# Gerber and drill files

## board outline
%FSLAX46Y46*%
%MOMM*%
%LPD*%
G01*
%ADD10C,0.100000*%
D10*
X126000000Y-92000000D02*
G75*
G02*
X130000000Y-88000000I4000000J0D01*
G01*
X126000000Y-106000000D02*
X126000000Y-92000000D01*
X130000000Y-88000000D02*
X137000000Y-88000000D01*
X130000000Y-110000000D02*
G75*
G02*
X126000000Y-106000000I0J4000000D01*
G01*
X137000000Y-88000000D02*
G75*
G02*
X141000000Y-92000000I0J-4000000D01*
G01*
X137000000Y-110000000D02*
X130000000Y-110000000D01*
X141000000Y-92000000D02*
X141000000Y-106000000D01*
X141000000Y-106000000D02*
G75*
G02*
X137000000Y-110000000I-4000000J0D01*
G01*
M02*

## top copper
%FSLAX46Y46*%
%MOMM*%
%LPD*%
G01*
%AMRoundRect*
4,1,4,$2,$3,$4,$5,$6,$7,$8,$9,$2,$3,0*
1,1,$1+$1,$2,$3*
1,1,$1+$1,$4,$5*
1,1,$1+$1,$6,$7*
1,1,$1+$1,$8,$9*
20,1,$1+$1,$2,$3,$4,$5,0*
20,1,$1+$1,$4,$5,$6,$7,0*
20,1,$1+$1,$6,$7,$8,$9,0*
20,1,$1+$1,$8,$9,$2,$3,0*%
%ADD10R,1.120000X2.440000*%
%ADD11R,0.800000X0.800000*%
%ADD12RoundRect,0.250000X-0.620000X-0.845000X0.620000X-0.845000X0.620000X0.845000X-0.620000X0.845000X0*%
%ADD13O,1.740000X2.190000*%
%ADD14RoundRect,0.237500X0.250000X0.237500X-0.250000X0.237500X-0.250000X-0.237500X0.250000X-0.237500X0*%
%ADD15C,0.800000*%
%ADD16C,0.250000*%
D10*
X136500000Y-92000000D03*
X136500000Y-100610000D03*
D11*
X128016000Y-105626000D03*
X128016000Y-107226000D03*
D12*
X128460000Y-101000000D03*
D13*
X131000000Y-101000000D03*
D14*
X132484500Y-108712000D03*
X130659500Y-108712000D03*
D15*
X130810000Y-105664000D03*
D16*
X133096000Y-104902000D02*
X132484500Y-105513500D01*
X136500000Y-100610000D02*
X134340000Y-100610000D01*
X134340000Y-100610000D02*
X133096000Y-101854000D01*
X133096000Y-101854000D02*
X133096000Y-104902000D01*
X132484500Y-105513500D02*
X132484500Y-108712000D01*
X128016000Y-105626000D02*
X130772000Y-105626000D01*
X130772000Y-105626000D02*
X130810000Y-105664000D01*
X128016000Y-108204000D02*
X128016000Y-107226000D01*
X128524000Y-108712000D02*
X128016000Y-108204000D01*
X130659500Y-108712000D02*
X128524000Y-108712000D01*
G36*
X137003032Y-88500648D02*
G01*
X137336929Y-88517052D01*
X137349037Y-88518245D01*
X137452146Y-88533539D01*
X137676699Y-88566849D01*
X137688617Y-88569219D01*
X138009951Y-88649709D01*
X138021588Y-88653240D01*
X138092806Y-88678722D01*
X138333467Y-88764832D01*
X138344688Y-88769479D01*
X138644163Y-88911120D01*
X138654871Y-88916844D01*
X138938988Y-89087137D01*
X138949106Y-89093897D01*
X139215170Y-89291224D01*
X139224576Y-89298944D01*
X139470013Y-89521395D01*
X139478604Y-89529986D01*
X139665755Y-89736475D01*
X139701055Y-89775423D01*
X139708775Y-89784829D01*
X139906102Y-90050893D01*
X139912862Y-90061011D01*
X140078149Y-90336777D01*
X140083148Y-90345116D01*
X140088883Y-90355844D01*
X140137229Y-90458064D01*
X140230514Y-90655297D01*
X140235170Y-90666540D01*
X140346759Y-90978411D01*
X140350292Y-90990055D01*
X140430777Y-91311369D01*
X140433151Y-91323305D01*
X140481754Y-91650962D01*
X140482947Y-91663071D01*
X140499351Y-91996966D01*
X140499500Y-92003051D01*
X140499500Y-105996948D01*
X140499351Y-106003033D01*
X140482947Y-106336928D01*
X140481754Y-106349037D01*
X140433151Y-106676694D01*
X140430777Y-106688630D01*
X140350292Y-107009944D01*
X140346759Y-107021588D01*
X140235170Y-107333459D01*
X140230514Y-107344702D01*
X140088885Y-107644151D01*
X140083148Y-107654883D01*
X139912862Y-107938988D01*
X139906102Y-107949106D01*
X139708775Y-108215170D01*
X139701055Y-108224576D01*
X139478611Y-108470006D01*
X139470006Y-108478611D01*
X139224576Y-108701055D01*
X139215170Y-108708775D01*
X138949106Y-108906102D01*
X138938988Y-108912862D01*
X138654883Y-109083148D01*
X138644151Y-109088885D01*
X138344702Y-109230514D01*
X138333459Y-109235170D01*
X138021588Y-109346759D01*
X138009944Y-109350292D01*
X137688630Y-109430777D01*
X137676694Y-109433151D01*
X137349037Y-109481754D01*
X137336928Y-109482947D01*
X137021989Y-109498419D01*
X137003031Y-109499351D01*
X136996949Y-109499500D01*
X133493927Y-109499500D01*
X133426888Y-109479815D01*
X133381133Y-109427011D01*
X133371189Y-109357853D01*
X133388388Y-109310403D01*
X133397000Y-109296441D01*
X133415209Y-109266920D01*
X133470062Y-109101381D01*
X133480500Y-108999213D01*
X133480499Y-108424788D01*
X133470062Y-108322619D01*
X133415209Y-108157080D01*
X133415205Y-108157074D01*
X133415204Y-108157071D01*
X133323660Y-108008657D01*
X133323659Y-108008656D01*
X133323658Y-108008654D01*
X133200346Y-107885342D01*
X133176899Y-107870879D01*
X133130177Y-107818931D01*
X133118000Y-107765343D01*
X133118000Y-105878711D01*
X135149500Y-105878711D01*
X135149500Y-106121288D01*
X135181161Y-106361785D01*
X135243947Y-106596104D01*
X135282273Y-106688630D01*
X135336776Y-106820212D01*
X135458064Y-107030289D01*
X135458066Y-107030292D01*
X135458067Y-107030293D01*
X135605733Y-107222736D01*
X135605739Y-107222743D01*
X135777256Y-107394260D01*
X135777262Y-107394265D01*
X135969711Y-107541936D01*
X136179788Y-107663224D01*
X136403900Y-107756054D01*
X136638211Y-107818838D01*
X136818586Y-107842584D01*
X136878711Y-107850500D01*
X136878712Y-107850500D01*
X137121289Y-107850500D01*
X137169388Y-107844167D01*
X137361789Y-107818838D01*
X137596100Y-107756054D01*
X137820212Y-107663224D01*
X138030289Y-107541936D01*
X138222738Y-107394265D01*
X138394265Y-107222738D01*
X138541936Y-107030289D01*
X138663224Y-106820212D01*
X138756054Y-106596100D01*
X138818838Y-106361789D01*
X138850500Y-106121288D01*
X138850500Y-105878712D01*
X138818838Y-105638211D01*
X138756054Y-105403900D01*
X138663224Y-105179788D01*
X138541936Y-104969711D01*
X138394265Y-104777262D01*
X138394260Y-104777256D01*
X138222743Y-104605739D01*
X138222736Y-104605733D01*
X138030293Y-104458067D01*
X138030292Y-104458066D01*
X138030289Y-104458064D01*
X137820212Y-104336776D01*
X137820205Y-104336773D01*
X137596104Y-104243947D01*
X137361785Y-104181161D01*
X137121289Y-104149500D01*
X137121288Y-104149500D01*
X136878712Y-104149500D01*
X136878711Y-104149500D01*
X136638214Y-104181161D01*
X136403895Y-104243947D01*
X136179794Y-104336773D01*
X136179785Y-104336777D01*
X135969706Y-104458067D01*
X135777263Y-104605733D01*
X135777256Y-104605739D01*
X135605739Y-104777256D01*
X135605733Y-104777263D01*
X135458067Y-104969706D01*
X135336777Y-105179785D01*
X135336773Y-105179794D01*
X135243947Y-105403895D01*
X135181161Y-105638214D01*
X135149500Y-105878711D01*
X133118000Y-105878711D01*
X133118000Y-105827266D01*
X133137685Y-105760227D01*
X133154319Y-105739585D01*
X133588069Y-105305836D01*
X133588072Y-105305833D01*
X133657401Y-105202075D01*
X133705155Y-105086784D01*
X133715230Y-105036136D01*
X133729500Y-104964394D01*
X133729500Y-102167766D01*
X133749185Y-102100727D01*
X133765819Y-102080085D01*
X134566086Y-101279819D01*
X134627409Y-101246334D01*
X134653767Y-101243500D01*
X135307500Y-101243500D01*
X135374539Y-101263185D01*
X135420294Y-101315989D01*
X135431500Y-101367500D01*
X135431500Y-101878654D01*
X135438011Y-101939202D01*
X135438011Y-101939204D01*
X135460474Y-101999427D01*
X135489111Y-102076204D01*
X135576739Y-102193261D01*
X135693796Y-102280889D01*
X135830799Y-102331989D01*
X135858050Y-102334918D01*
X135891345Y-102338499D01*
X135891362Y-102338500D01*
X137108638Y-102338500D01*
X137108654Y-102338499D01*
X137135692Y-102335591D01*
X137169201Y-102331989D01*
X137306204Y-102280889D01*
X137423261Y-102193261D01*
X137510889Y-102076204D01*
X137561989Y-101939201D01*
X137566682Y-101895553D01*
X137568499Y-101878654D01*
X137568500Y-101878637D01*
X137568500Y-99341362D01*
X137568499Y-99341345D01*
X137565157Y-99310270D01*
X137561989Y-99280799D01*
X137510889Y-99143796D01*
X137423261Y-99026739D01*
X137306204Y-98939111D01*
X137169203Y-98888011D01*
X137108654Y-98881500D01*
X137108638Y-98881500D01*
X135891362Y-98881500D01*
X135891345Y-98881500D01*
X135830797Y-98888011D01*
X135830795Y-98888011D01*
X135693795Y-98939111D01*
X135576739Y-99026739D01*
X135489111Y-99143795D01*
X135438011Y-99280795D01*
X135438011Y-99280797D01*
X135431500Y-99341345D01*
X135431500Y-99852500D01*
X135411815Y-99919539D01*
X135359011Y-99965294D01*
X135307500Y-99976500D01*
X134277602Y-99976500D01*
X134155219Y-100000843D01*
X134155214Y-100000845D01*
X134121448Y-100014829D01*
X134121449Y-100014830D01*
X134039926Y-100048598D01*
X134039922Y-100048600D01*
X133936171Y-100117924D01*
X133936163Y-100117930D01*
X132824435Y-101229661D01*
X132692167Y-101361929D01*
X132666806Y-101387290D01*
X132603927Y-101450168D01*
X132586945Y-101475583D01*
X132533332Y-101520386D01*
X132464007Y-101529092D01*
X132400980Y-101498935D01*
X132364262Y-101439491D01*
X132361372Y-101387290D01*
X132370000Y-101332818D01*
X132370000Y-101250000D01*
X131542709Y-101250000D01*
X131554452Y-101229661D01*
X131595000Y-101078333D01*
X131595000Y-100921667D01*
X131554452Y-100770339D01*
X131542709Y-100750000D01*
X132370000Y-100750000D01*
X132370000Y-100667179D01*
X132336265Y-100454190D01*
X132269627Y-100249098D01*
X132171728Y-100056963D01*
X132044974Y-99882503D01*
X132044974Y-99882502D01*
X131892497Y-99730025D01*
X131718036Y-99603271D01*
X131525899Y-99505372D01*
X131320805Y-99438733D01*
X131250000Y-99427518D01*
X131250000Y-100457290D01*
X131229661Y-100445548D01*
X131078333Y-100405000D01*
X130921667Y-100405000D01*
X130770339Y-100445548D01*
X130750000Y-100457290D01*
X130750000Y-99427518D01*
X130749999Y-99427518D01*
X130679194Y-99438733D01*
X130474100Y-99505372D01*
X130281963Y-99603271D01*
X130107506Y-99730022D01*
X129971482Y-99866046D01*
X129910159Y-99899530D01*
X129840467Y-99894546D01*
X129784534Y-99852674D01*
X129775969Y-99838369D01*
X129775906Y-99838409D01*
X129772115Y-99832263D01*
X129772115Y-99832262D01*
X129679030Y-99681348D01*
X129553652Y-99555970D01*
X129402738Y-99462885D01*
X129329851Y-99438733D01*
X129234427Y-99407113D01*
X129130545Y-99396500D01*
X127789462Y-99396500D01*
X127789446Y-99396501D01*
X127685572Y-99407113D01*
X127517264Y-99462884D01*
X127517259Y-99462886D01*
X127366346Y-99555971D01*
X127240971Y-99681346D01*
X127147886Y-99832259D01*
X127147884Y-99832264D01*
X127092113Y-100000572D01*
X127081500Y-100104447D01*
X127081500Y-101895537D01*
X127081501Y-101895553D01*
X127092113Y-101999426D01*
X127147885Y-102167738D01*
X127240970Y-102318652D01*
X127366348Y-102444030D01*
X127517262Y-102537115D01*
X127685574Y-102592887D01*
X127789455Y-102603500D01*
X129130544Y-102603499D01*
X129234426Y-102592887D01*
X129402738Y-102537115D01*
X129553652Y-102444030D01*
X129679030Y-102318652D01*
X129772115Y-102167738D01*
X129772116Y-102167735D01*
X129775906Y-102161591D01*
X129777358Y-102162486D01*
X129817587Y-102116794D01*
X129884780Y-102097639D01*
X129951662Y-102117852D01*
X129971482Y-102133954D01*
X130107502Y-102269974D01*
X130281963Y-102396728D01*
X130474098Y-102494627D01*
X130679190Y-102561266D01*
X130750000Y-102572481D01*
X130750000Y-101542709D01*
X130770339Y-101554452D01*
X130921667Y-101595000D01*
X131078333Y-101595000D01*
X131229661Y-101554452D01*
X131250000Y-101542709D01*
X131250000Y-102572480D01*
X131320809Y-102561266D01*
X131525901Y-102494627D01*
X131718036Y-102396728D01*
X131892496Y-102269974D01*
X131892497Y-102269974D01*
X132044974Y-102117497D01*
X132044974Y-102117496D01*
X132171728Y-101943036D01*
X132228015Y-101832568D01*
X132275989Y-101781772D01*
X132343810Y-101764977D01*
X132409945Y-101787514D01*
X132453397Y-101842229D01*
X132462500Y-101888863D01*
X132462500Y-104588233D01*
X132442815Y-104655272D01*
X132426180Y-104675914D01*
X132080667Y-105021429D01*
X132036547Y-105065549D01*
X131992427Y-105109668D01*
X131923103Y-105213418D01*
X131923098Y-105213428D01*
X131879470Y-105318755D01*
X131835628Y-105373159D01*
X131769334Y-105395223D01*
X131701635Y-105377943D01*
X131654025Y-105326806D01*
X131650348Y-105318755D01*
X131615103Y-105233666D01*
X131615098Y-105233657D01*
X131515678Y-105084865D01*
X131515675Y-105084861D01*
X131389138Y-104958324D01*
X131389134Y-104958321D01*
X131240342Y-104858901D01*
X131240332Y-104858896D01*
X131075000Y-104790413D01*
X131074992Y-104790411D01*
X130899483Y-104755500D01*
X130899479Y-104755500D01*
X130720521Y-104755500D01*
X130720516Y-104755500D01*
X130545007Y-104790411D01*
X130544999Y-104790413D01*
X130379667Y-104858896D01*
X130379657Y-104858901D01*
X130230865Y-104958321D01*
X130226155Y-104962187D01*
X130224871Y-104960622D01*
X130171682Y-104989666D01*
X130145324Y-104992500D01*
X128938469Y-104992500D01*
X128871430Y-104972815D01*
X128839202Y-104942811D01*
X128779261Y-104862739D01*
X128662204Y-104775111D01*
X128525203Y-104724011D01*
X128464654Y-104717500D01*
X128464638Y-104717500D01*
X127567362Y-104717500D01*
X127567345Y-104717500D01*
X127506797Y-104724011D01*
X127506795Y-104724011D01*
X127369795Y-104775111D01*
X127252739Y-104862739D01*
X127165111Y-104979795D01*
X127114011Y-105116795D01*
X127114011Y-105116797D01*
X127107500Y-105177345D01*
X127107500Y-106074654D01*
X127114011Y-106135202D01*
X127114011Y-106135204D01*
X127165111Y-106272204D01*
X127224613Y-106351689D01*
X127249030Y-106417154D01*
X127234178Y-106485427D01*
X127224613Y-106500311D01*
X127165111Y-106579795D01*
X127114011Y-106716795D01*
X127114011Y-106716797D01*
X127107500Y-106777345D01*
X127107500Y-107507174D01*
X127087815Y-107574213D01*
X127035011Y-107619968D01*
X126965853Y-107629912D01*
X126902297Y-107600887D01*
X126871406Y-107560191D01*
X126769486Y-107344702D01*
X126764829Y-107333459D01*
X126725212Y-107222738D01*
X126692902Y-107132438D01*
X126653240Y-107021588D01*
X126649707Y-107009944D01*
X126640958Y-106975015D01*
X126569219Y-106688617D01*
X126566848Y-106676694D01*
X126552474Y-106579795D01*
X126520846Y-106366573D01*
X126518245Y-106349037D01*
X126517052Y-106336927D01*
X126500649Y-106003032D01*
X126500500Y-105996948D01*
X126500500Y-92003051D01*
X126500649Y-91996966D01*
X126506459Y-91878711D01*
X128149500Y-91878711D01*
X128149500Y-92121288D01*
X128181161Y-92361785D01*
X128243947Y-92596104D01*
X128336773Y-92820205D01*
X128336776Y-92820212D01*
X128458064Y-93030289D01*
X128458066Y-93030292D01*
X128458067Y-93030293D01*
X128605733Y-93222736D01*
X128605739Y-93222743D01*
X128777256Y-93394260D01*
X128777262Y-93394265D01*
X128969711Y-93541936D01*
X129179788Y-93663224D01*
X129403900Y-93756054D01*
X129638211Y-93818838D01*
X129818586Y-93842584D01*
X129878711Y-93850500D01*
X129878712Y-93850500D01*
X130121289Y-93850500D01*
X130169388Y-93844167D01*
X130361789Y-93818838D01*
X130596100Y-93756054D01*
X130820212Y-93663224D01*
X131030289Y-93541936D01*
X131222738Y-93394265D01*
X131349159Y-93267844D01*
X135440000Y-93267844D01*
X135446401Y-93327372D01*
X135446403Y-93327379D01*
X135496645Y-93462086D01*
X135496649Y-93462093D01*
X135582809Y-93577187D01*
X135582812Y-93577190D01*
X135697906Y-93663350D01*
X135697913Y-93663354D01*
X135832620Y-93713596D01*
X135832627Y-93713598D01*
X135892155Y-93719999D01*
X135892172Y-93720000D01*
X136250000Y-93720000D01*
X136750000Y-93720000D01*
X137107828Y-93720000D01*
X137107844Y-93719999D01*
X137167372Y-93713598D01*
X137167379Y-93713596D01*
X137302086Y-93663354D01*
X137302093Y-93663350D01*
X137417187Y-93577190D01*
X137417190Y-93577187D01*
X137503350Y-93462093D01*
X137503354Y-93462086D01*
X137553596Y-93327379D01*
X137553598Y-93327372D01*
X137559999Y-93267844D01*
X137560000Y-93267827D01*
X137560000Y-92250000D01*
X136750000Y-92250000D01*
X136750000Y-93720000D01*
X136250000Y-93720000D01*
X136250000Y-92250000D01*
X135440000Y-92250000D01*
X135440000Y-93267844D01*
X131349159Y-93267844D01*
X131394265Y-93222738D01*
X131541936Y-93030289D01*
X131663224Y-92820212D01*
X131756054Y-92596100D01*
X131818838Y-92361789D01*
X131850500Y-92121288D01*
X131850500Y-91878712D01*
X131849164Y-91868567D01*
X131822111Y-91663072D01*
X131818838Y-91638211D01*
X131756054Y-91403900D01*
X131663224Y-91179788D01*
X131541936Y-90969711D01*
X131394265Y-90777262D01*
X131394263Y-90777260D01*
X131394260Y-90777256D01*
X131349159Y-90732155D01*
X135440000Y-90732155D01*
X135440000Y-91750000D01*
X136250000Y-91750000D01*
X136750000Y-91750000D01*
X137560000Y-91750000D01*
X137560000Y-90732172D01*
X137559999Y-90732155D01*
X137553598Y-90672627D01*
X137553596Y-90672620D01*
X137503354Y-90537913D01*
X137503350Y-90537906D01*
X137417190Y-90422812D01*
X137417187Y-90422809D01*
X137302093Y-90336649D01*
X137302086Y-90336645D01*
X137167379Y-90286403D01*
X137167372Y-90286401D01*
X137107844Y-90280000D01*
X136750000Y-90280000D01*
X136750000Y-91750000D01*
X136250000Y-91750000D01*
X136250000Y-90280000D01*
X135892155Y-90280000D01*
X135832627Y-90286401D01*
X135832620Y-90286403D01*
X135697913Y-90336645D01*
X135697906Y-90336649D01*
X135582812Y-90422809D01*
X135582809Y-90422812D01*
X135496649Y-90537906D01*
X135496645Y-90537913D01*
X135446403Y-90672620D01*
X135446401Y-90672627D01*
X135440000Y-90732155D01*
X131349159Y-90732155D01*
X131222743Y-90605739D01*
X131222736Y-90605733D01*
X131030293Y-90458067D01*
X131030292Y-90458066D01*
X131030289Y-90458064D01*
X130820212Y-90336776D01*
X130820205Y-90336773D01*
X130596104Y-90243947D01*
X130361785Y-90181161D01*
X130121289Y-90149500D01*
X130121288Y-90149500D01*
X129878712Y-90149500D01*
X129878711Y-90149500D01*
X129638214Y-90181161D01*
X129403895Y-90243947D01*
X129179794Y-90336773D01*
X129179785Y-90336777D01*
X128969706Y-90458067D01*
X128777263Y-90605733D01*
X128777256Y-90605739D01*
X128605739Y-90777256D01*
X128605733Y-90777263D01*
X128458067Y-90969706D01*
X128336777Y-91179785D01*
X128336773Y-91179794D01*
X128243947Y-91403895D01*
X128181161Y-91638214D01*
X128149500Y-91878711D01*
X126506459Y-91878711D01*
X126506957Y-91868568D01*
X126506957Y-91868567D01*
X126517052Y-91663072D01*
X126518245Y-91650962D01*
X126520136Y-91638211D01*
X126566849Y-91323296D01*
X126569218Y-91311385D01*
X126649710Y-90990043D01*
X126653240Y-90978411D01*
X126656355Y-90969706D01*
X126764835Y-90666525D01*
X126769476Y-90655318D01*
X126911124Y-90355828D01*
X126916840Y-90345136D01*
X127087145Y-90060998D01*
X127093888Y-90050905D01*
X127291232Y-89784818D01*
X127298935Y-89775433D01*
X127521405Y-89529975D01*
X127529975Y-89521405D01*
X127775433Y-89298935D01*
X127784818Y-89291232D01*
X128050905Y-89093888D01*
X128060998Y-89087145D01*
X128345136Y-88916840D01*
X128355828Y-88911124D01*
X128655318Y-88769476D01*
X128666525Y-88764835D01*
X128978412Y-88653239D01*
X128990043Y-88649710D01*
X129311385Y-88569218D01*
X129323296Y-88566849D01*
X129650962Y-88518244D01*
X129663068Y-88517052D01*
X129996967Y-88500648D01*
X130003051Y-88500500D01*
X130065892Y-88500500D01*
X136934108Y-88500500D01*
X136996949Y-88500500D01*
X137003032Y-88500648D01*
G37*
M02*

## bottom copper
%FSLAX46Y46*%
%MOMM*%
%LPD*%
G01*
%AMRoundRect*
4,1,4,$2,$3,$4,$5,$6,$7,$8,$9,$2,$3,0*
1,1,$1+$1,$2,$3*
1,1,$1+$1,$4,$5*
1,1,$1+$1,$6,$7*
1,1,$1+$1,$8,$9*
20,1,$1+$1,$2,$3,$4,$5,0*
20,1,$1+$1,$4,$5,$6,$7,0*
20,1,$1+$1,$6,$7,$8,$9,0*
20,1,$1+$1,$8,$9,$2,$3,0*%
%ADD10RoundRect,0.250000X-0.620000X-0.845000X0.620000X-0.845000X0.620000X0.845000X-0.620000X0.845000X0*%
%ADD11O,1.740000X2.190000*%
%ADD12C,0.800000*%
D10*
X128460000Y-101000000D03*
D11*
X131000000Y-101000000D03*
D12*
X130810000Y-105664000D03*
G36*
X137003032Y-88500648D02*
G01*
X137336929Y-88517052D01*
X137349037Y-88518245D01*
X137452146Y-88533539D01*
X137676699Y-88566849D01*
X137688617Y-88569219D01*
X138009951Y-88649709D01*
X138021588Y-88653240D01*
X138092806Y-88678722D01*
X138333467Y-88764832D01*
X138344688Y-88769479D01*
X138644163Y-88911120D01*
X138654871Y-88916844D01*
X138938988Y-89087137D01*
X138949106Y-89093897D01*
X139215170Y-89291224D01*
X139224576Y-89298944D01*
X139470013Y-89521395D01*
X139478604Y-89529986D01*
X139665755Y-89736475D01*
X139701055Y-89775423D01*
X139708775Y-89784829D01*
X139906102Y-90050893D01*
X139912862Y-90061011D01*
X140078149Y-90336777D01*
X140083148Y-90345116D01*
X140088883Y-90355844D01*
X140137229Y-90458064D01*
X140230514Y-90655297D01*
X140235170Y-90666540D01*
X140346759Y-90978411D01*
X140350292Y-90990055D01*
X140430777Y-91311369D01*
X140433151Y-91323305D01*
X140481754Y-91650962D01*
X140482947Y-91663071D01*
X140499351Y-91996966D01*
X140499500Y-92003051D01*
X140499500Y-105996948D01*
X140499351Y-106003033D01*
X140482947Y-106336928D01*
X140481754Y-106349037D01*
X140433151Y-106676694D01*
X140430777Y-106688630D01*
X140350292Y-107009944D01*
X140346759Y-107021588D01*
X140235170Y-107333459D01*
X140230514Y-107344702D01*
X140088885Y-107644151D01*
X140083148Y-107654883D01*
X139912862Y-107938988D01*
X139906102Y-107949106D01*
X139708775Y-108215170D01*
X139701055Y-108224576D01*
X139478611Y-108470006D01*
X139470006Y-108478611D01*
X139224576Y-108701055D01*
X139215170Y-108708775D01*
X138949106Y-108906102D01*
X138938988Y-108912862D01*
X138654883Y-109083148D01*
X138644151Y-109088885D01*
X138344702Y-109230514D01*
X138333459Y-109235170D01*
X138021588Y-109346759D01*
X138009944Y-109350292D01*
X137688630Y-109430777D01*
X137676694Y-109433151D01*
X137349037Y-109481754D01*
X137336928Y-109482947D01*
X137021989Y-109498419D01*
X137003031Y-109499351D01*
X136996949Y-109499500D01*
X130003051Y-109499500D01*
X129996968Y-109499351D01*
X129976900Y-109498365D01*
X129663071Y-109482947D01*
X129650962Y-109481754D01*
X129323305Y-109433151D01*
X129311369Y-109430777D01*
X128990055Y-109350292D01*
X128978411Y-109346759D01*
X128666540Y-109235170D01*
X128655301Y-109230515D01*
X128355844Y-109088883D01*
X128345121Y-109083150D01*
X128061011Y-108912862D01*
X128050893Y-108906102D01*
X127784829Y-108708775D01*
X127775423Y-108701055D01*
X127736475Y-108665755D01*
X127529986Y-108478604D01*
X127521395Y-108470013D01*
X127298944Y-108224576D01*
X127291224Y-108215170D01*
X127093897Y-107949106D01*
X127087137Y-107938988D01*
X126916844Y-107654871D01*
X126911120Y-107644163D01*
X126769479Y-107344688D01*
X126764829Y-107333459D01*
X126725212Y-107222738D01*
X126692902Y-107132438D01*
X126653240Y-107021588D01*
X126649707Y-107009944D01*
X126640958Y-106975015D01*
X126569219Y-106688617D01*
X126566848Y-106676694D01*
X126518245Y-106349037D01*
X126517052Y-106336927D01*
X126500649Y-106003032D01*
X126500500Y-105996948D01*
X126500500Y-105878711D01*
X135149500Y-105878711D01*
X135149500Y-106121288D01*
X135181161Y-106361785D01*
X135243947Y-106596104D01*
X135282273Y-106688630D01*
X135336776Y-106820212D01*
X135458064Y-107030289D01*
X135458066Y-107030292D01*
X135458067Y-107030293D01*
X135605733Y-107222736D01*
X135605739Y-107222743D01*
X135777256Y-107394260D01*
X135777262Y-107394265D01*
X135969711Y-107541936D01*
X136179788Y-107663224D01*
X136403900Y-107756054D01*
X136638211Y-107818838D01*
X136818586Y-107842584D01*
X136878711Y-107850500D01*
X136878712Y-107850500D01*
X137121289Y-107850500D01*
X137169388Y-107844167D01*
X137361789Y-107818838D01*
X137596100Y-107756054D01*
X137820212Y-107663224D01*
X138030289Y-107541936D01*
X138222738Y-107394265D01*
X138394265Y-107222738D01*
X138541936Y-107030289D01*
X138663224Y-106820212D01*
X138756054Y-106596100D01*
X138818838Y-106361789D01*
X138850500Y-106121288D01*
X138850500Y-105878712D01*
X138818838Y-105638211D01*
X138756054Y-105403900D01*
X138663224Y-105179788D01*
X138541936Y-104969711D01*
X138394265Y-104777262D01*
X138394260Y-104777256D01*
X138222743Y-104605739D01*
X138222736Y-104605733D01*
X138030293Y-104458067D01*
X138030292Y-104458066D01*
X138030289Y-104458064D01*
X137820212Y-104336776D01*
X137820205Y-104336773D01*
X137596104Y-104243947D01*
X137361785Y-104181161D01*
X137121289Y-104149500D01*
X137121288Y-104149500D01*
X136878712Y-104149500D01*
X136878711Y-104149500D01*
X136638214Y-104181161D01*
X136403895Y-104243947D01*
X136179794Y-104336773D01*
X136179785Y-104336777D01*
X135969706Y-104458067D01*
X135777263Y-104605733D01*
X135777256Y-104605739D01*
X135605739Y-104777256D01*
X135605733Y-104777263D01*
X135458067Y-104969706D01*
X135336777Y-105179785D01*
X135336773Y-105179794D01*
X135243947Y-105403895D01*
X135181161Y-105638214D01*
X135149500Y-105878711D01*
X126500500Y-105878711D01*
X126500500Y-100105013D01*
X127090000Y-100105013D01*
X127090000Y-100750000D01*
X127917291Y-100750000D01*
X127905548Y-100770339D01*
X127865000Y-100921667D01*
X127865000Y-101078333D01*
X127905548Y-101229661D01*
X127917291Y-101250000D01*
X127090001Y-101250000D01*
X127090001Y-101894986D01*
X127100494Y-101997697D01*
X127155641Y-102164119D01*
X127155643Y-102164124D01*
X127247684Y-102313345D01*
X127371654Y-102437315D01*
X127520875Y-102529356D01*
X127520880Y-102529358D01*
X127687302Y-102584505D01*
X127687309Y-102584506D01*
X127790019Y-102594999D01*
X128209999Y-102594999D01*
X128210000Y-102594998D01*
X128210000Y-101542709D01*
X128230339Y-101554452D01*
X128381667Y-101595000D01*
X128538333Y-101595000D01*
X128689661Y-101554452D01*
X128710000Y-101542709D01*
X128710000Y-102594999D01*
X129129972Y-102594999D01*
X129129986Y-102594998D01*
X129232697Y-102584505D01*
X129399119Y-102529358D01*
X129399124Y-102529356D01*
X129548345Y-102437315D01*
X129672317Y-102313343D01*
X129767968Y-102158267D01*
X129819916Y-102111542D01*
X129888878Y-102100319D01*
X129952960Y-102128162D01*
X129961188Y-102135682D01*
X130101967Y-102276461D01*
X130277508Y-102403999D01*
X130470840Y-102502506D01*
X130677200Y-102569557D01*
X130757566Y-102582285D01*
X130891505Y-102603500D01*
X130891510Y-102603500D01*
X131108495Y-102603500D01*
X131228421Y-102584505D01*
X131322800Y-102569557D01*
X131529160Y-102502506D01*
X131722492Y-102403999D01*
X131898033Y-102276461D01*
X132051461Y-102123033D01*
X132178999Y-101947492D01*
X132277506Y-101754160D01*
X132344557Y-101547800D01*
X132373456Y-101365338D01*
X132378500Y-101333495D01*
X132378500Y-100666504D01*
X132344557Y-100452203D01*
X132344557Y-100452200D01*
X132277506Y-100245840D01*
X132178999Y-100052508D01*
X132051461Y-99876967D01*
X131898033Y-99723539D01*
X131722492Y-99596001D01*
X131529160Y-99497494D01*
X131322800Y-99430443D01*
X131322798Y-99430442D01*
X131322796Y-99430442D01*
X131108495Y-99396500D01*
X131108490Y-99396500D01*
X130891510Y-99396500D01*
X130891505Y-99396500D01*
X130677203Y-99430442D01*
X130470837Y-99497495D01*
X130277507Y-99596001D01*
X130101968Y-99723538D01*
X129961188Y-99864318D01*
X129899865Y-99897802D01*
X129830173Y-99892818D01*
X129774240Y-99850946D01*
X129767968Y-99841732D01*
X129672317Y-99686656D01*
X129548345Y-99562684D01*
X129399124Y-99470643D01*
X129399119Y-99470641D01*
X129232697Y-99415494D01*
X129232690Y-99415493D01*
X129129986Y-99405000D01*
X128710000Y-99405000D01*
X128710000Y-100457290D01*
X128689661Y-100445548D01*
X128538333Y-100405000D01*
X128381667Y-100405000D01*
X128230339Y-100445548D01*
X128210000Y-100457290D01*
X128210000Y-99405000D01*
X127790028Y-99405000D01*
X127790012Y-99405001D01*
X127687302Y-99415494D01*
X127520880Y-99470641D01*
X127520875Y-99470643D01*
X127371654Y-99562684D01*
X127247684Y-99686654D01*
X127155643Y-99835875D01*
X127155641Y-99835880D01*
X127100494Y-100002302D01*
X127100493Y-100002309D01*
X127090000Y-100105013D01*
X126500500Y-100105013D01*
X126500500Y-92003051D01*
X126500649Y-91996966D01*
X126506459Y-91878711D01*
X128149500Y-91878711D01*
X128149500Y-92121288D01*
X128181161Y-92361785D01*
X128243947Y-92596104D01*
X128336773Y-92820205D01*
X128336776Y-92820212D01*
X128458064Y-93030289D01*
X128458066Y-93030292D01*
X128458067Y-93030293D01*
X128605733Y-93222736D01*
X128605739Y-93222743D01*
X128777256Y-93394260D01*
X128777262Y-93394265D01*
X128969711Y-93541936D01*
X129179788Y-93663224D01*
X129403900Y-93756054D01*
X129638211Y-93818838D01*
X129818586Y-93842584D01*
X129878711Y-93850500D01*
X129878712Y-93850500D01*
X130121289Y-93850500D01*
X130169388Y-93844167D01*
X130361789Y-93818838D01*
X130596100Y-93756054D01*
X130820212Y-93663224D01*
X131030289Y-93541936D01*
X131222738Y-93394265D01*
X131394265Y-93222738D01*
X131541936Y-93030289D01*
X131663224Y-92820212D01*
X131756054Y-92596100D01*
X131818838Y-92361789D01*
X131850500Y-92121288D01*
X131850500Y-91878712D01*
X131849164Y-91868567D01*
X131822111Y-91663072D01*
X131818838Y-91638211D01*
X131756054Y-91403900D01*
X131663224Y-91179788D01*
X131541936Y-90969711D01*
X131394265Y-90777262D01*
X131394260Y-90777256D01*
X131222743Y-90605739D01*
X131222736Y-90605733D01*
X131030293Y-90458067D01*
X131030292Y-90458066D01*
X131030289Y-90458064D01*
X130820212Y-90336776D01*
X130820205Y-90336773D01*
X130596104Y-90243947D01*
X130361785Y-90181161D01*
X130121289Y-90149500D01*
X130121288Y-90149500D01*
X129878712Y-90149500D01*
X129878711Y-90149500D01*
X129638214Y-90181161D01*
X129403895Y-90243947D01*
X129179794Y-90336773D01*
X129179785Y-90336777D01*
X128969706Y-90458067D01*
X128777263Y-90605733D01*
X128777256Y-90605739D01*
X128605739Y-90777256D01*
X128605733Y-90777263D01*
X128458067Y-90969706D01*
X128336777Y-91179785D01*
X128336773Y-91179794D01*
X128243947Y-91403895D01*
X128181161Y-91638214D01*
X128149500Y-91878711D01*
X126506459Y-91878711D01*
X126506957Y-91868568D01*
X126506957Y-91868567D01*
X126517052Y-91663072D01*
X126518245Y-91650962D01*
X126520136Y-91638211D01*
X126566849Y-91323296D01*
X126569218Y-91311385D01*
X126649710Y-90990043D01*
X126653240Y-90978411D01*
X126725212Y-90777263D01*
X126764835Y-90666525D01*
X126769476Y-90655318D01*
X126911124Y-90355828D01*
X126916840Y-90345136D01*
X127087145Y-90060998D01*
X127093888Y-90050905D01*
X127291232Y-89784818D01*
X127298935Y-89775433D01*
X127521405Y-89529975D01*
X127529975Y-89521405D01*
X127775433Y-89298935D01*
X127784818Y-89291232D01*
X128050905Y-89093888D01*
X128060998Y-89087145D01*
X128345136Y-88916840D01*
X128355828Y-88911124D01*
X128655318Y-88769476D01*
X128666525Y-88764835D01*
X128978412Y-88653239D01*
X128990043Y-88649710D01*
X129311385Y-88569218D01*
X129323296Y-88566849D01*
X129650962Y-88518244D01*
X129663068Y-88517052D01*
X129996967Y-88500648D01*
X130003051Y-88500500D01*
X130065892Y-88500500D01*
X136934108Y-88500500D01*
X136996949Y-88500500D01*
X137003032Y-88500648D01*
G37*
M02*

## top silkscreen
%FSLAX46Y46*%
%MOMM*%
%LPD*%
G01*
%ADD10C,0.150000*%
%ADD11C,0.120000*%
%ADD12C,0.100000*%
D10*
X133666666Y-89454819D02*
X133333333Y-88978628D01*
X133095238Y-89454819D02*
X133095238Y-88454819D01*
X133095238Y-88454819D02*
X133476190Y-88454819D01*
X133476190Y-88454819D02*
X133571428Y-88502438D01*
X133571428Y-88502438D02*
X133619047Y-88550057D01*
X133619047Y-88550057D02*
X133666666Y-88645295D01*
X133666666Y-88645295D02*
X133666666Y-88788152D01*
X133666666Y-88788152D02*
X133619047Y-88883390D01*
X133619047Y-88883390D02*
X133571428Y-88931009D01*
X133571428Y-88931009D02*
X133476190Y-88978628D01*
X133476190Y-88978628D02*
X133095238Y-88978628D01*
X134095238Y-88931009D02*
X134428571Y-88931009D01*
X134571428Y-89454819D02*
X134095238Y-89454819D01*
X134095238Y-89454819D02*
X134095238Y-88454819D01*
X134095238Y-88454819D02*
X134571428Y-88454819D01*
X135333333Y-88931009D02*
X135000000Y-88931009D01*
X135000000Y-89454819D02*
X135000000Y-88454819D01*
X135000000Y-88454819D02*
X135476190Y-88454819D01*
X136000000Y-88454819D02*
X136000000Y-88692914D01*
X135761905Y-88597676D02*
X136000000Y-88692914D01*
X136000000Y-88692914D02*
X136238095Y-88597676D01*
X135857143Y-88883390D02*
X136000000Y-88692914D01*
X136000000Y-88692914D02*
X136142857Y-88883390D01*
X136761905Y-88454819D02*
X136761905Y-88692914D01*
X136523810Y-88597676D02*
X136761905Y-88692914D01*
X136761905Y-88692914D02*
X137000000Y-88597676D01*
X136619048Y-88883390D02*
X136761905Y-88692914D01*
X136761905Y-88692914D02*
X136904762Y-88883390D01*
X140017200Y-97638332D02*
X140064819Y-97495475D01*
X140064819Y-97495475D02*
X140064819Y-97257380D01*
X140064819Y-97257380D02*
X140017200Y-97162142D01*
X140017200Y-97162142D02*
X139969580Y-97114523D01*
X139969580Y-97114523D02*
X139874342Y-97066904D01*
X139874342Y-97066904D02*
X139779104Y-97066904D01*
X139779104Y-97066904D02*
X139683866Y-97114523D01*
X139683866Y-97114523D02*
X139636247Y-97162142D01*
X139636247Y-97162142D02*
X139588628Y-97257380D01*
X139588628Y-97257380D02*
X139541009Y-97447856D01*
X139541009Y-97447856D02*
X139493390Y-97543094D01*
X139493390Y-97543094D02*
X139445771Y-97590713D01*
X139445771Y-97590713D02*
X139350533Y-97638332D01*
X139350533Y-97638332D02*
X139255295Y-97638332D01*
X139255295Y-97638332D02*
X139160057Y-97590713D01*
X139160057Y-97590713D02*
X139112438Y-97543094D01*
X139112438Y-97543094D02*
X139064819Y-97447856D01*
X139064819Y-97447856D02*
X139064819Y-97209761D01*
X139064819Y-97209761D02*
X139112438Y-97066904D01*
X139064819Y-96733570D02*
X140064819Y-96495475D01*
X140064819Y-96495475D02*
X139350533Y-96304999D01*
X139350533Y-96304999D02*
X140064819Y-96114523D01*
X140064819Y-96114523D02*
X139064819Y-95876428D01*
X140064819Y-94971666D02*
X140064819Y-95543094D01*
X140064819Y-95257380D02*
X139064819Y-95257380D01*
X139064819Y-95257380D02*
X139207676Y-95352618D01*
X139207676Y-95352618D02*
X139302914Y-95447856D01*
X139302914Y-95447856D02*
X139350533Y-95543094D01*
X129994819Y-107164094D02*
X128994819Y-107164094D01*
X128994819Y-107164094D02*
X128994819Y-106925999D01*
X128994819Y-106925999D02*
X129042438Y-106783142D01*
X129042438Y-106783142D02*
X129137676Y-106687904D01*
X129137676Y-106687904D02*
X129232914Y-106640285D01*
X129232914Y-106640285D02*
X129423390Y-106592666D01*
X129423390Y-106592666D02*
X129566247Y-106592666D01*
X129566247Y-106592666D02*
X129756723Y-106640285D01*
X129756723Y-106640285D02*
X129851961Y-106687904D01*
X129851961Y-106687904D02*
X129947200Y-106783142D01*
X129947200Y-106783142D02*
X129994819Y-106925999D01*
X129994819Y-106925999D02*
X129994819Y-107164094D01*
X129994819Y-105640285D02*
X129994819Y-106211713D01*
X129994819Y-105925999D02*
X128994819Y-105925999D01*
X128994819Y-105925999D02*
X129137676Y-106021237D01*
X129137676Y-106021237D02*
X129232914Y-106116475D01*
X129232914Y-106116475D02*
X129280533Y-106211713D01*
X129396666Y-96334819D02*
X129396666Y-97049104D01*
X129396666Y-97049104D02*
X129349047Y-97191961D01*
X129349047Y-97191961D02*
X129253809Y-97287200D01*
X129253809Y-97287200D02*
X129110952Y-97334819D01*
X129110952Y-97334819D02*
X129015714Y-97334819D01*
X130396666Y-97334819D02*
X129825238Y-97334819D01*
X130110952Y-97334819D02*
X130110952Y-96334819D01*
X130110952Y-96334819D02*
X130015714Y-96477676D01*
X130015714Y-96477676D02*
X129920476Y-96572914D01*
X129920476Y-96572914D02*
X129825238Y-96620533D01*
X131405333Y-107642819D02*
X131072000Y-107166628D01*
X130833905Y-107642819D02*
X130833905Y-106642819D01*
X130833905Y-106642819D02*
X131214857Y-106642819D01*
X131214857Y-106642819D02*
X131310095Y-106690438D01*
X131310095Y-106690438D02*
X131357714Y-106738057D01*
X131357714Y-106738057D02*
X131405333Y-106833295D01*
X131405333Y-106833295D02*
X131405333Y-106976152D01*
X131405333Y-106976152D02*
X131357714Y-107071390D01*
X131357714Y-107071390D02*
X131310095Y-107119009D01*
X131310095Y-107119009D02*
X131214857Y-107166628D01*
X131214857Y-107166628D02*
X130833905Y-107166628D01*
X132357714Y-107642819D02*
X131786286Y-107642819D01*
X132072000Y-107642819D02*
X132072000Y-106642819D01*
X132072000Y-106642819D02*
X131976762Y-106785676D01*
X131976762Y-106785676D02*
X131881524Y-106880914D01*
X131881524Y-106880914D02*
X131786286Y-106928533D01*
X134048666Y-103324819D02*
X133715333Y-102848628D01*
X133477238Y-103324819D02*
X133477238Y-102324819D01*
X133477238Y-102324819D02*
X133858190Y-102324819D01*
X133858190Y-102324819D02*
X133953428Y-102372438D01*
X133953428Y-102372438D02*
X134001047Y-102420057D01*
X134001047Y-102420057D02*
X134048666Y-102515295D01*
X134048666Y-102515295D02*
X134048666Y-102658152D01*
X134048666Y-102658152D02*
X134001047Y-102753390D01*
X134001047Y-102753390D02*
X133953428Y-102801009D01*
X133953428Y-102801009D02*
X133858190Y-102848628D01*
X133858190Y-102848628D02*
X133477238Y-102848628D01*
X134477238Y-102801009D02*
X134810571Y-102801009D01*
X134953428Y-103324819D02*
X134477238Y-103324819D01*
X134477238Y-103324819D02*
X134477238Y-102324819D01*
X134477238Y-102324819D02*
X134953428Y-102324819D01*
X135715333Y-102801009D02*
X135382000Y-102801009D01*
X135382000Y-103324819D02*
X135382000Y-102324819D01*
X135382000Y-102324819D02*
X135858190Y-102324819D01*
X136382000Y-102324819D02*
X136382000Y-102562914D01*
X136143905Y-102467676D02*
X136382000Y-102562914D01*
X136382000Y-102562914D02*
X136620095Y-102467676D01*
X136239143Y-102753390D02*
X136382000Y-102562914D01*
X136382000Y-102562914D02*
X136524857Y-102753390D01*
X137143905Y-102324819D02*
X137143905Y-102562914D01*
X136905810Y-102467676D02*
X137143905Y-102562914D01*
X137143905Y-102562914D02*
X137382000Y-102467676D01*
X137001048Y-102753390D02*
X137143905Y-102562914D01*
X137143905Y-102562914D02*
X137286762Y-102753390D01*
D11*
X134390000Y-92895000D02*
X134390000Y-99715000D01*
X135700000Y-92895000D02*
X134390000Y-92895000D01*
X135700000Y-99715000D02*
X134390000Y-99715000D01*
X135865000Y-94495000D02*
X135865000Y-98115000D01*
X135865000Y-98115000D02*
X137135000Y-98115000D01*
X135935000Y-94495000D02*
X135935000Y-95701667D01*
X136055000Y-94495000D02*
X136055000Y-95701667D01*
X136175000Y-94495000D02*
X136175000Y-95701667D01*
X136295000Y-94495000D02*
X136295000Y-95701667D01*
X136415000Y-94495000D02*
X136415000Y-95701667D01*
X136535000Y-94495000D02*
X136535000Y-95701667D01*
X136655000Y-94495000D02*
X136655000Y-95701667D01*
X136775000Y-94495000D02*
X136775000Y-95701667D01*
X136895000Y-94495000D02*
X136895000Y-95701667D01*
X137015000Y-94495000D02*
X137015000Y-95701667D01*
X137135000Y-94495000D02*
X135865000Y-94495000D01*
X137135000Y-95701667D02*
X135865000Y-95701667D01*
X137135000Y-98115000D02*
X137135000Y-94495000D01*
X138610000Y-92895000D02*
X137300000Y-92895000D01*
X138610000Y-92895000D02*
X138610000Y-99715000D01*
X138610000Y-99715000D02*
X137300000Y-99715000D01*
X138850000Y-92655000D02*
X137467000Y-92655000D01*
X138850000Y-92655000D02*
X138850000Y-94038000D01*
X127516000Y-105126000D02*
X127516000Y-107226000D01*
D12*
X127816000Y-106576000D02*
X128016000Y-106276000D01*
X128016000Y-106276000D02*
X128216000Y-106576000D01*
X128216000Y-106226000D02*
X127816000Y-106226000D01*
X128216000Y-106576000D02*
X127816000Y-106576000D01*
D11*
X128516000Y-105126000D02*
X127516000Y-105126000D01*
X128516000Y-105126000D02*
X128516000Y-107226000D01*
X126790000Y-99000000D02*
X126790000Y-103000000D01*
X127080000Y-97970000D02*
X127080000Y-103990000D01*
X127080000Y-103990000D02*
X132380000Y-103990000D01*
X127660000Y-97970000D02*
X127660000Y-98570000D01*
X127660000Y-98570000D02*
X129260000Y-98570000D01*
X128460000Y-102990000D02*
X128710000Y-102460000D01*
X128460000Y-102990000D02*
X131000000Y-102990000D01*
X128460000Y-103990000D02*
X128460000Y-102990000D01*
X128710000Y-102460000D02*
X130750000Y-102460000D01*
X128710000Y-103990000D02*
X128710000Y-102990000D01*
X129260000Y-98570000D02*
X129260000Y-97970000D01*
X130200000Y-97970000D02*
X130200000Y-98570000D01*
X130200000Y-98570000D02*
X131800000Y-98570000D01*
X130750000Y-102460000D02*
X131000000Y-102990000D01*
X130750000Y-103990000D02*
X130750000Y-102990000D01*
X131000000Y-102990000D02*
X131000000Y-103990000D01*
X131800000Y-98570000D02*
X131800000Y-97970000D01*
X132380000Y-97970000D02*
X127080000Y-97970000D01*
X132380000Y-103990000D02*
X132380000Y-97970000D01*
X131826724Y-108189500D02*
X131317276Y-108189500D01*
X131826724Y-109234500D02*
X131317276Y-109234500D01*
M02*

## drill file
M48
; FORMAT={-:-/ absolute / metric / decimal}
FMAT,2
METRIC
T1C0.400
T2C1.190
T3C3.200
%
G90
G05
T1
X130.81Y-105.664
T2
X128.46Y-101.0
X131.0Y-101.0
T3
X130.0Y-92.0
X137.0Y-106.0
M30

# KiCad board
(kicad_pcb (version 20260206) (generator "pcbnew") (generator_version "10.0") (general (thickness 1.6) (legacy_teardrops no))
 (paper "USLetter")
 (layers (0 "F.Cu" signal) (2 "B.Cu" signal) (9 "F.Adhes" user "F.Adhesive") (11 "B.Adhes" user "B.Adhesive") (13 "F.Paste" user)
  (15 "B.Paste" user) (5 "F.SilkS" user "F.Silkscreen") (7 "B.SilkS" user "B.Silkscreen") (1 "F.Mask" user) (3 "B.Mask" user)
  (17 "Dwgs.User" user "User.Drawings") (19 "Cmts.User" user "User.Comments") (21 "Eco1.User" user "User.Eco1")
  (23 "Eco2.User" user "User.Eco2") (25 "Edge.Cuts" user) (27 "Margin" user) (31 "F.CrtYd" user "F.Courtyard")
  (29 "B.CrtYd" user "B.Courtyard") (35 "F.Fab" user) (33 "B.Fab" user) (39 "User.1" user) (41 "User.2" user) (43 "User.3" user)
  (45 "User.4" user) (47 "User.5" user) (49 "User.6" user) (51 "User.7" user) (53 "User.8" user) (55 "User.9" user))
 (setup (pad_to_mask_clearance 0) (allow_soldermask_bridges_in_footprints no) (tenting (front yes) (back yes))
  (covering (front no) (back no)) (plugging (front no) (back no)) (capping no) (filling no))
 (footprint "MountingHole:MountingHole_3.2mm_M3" (layer "F.Cu") (at 130 92)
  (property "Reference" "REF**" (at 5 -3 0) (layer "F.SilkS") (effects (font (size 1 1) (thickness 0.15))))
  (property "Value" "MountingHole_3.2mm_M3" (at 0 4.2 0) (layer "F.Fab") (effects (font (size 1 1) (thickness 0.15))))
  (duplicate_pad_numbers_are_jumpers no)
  (pad "" np_thru_hole circle (at 0 0) (size 3.2 3.2) (drill 3.2) (layers "*.Cu" "*.Mask")))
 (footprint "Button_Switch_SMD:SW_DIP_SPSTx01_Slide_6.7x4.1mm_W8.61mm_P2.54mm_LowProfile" (layer "F.Cu") (at 136.5 96.305 -90)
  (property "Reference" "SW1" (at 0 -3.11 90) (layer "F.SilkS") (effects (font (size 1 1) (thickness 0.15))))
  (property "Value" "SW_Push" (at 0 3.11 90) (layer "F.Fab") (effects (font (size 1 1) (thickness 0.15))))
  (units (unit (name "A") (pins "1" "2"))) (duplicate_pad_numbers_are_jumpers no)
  (fp_line (start -3.41 2.11) (end 3.41 2.11) (stroke (width 0.12) (type solid)) (layer "F.SilkS"))
  (fp_line (start -3.41 0.8) (end -3.41 2.11) (stroke (width 0.12) (type solid)) (layer "F.SilkS"))
  (fp_line (start 3.41 0.8) (end 3.41 2.11) (stroke (width 0.12) (type solid)) (layer "F.SilkS"))
  (fp_line (start -1.81 0.635) (end 1.81 0.635) (stroke (width 0.12) (type solid)) (layer "F.SilkS"))
  (fp_line (start 1.81 0.635) (end 1.81 -0.635) (stroke (width 0.12) (type solid)) (layer "F.SilkS"))
  (fp_line (start -1.81 0.565) (end -0.603333 0.565) (stroke (width 0.12) (type solid)) (layer "F.SilkS"))
  (fp_line (start -1.81 0.445) (end -0.603333 0.445) (stroke (width 0.12) (type solid)) (layer "F.SilkS"))
  (fp_line (start -1.81 0.325) (end -0.603333 0.325) (stroke (width 0.12) (type solid)) (layer "F.SilkS"))
  (fp_line (start -1.81 0.205) (end -0.603333 0.205) (stroke (width 0.12) (type solid)) (layer "F.SilkS"))
  (fp_line (start -1.81 0.085) (end -0.603333 0.085) (stroke (width 0.12) (type solid)) (layer "F.SilkS"))
  (fp_line (start -1.81 -0.035) (end -0.603333 -0.035) (stroke (width 0.12) (type solid)) (layer "F.SilkS"))
  (fp_line (start -1.81 -0.155) (end -0.603333 -0.155) (stroke (width 0.12) (type solid)) (layer "F.SilkS"))
  (fp_line (start -1.81 -0.275) (end -0.603333 -0.275) (stroke (width 0.12) (type solid)) (layer "F.SilkS"))
  (fp_line (start -1.81 -0.395) (end -0.603333 -0.395) (stroke (width 0.12) (type solid)) (layer "F.SilkS"))
  (fp_line (start -1.81 -0.515) (end -0.603333 -0.515) (stroke (width 0.12) (type solid)) (layer "F.SilkS"))
  (fp_line (start -1.81 -0.635) (end -1.81 0.635) (stroke (width 0.12) (type solid)) (layer "F.SilkS"))
  (fp_line (start -0.603333 -0.635) (end -0.603333 0.635) (stroke (width 0.12) (type solid)) (layer "F.SilkS"))
  (fp_line (start 1.81 -0.635) (end -1.81 -0.635) (stroke (width 0.12) (type solid)) (layer "F.SilkS"))
  (fp_line (start -3.41 -2.11) (end -3.41 -0.8) (stroke (width 0.12) (type solid)) (layer "F.SilkS"))
  (fp_line (start -3.41 -2.11) (end 3.41 -2.11) (stroke (width 0.12) (type solid)) (layer "F.SilkS"))
  (fp_line (start 3.41 -2.11) (end 3.41 -0.8) (stroke (width 0.12) (type solid)) (layer "F.SilkS"))
  (fp_line (start -3.65 -2.35) (end -3.65 -0.967) (stroke (width 0.12) (type solid)) (layer "F.SilkS"))
  (fp_line (start -3.65 -2.35) (end -2.267 -2.35) (stroke (width 0.12) (type solid)) (layer "F.SilkS"))
  (pad "1" smd rect (at -4.305 0 270) (size 2.44 1.12) (layers "F.Cu" "F.Mask" "F.Paste") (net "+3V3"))
  (pad "2" smd rect (at 4.305 0 270) (size 2.44 1.12) (layers "F.Cu" "F.Mask" "F.Paste") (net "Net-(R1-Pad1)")))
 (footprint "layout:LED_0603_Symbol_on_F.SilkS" (layer "F.Cu") (at 128.016 106.426 -90)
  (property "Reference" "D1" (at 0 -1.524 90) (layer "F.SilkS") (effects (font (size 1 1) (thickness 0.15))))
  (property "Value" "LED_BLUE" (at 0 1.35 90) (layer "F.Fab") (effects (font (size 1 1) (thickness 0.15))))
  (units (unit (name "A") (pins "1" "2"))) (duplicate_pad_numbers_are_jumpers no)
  (fp_line (start -1.3 0.5) (end 0.8 0.5) (stroke (width 0.12) (type solid)) (layer "F.SilkS"))
  (fp_line (start 0.15 0.2) (end -0.15 0) (stroke (width 0.1) (type solid)) (layer "F.SilkS"))
  (fp_line (start -0.15 0) (end 0.15 -0.2) (stroke (width 0.1) (type solid)) (layer "F.SilkS"))
  (fp_line (start -0.2 -0.2) (end -0.2 0.2) (stroke (width 0.1) (type solid)) (layer "F.SilkS"))
  (fp_line (start 0.15 -0.2) (end 0.15 0.2) (stroke (width 0.1) (type solid)) (layer "F.SilkS"))
  (fp_line (start -1.3 -0.5) (end -1.3 0.5) (stroke (width 0.12) (type solid)) (layer "F.SilkS"))
  (fp_line (start -1.3 -0.5) (end 0.8 -0.5) (stroke (width 0.12) (type solid)) (layer "F.SilkS"))
  (pad "1" smd rect (at -0.8 0 90) (size 0.8 0.8) (layers "F.Cu" "F.Mask" "F.Paste") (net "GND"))
  (pad "2" smd rect (at 0.8 0 90) (size 0.8 0.8) (layers "F.Cu" "F.Mask" "F.Paste") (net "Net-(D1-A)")))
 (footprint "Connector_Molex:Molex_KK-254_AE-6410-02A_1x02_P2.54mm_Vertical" (layer "F.Cu") (at 128.46 101)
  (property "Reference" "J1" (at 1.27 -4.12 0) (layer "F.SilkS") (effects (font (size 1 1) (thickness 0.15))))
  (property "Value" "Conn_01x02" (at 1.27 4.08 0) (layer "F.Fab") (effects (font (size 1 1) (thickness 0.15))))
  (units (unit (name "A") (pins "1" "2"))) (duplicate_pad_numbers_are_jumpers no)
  (fp_line (start -1.67 -2) (end -1.67 2) (stroke (width 0.12) (type solid)) (layer "F.SilkS"))
  (fp_line (start -1.38 -3.03) (end -1.38 2.99) (stroke (width 0.12) (type solid)) (layer "F.SilkS"))
  (fp_line (start -1.38 2.99) (end 3.92 2.99) (stroke (width 0.12) (type solid)) (layer "F.SilkS"))
  (fp_line (start -0.8 -3.03) (end -0.8 -2.43) (stroke (width 0.12) (type solid)) (layer "F.SilkS"))
  (fp_line (start -0.8 -2.43) (end 0.8 -2.43) (stroke (width 0.12) (type solid)) (layer "F.SilkS"))
  (fp_line (start 0 1.99) (end 0.25 1.46) (stroke (width 0.12) (type solid)) (layer "F.SilkS"))
  (fp_line (start 0 1.99) (end 2.54 1.99) (stroke (width 0.12) (type solid)) (layer "F.SilkS"))
  (fp_line (start 0 2.99) (end 0 1.99) (stroke (width 0.12) (type solid)) (layer "F.SilkS"))
  (fp_line (start 0.25 1.46) (end 2.29 1.46) (stroke (width 0.12) (type solid)) (layer "F.SilkS"))
  (fp_line (start 0.25 2.99) (end 0.25 1.99) (stroke (width 0.12) (type solid)) (layer "F.SilkS"))
  (fp_line (start 0.8 -2.43) (end 0.8 -3.03) (stroke (width 0.12) (type solid)) (layer "F.SilkS"))
  (fp_line (start 1.74 -3.03) (end 1.74 -2.43) (stroke (width 0.12) (type solid)) (layer "F.SilkS"))
  (fp_line (start 1.74 -2.43) (end 3.34 -2.43) (stroke (width 0.12) (type solid)) (layer "F.SilkS"))
  (fp_line (start 2.29 1.46) (end 2.54 1.99) (stroke (width 0.12) (type solid)) (layer "F.SilkS"))
  (fp_line (start 2.29 2.99) (end 2.29 1.99) (stroke (width 0.12) (type solid)) (layer "F.SilkS"))
  (fp_line (start 2.54 1.99) (end 2.54 2.99) (stroke (width 0.12) (type solid)) (layer "F.SilkS"))
  (fp_line (start 3.34 -2.43) (end 3.34 -3.03) (stroke (width 0.12) (type solid)) (layer "F.SilkS"))
  (fp_line (start 3.92 -3.03) (end -1.38 -3.03) (stroke (width 0.12) (type solid)) (layer "F.SilkS"))
  (fp_line (start 3.92 2.99) (end 3.92 -3.03) (stroke (width 0.12) (type solid)) (layer "F.SilkS"))
  (pad "1" thru_hole roundrect (at 0 0) (size 1.74 2.19) (drill 1.19) (layers "*.Cu" "*.Mask") (remove_unused_layers no)
   (roundrect_rratio 0.143678) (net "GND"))
  (pad "2" thru_hole oval (at 2.54 0) (size 1.74 2.19) (drill 1.19) (layers "*.Cu" "*.Mask") (remove_unused_layers no) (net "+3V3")))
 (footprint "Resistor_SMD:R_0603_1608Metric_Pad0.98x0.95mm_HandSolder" (layer "F.Cu") (at 131.572 108.712 180)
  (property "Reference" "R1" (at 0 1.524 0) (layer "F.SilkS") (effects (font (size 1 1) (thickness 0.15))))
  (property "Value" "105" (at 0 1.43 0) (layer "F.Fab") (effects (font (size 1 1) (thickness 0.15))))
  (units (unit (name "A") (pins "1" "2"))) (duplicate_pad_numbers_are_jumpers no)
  (fp_line (start -0.254724 0.5225) (end 0.254724 0.5225) (stroke (width 0.12) (type solid)) (layer "F.SilkS"))
  (fp_line (start -0.254724 -0.5225) (end 0.254724 -0.5225) (stroke (width 0.12) (type solid)) (layer "F.SilkS"))
  (pad "1" smd roundrect (at -0.9125 0 180) (size 0.975 0.95) (layers "F.Cu" "F.Mask" "F.Paste") (roundrect_rratio 0.25)
   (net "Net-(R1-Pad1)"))
  (pad "2" smd roundrect (at 0.9125 0 180) (size 0.975 0.95) (layers "F.Cu" "F.Mask" "F.Paste") (roundrect_rratio 0.25) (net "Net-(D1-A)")))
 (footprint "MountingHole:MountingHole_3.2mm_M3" (layer "F.Cu") (at 137 106)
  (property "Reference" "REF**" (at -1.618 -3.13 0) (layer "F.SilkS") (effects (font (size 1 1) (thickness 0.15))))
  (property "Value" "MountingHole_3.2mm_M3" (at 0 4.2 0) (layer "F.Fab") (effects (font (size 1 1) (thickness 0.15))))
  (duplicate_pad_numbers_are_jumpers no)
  (pad "" np_thru_hole circle (at 0 0) (size 3.2 3.2) (drill 3.2) (layers "*.Cu" "*.Mask")))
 (gr_arc (start 126 92) (mid 127.171573 89.171573) (end 130 88) (stroke (width 0.1) (type default)) (layer "Edge.Cuts"))
 (gr_line (start 126 106) (end 126 92) (stroke (width 0.1) (type default)) (layer "Edge.Cuts"))
 (gr_line (start 130 88) (end 137 88) (stroke (width 0.1) (type default)) (layer "Edge.Cuts"))
 (gr_arc (start 130 110) (mid 127.171573 108.828427) (end 126 106) (stroke (width 0.1) (type default)) (layer "Edge.Cuts"))
 (gr_arc (start 137 88) (mid 139.828427 89.171573) (end 141 92) (stroke (width 0.1) (type default)) (layer "Edge.Cuts"))
 (gr_line (start 137 110) (end 130 110) (stroke (width 0.1) (type default)) (layer "Edge.Cuts"))
 (gr_line (start 141 92) (end 141 106) (stroke (width 0.1) (type default)) (layer "Edge.Cuts"))
 (gr_arc (start 141 106) (mid 139.828427 108.828427) (end 137 110) (stroke (width 0.1) (type default)) (layer "Edge.Cuts"))
 (segment (start 133.096 104.902) (end 132.4845 105.5135) (width 0.25) (layer "F.Cu") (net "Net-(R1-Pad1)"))
 (segment (start 136.5 100.61) (end 134.34 100.61) (width 0.25) (layer "F.Cu") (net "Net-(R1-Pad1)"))
 (segment (start 134.34 100.61) (end 133.096 101.854) (width 0.25) (layer "F.Cu") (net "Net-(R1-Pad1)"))
 (segment (start 133.096 101.854) (end 133.096 104.902) (width 0.25) (layer "F.Cu") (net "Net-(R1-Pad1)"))
 (segment (start 132.4845 105.5135) (end 132.4845 108.712) (width 0.25) (layer "F.Cu") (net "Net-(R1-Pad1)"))
 (segment (start 128.016 105.626) (end 130.772 105.626) (width 0.25) (layer "F.Cu") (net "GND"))
 (segment (start 130.772 105.626) (end 130.81 105.664) (width 0.25) (layer "F.Cu") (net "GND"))
 (via (at 130.81 105.664) (size 0.8) (drill 0.4) (layers "F.Cu" "B.Cu") (free yes) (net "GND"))
 (segment (start 128.016 108.204) (end 128.016 107.226) (width 0.25) (layer "F.Cu") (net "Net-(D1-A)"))
 (segment (start 128.524 108.712) (end 128.016 108.204) (width 0.25) (layer "F.Cu") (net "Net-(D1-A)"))
 (segment (start 130.6595 108.712) (end 128.524 108.712) (width 0.25) (layer "F.Cu") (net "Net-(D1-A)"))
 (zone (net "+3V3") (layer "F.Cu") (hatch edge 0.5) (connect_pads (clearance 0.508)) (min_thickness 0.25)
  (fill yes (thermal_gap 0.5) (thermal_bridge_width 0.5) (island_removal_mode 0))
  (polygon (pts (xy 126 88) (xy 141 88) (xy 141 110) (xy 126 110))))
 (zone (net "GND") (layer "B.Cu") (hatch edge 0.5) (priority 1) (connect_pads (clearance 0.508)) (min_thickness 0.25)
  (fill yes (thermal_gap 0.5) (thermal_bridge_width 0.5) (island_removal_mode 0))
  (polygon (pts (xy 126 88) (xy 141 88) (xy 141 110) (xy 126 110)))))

